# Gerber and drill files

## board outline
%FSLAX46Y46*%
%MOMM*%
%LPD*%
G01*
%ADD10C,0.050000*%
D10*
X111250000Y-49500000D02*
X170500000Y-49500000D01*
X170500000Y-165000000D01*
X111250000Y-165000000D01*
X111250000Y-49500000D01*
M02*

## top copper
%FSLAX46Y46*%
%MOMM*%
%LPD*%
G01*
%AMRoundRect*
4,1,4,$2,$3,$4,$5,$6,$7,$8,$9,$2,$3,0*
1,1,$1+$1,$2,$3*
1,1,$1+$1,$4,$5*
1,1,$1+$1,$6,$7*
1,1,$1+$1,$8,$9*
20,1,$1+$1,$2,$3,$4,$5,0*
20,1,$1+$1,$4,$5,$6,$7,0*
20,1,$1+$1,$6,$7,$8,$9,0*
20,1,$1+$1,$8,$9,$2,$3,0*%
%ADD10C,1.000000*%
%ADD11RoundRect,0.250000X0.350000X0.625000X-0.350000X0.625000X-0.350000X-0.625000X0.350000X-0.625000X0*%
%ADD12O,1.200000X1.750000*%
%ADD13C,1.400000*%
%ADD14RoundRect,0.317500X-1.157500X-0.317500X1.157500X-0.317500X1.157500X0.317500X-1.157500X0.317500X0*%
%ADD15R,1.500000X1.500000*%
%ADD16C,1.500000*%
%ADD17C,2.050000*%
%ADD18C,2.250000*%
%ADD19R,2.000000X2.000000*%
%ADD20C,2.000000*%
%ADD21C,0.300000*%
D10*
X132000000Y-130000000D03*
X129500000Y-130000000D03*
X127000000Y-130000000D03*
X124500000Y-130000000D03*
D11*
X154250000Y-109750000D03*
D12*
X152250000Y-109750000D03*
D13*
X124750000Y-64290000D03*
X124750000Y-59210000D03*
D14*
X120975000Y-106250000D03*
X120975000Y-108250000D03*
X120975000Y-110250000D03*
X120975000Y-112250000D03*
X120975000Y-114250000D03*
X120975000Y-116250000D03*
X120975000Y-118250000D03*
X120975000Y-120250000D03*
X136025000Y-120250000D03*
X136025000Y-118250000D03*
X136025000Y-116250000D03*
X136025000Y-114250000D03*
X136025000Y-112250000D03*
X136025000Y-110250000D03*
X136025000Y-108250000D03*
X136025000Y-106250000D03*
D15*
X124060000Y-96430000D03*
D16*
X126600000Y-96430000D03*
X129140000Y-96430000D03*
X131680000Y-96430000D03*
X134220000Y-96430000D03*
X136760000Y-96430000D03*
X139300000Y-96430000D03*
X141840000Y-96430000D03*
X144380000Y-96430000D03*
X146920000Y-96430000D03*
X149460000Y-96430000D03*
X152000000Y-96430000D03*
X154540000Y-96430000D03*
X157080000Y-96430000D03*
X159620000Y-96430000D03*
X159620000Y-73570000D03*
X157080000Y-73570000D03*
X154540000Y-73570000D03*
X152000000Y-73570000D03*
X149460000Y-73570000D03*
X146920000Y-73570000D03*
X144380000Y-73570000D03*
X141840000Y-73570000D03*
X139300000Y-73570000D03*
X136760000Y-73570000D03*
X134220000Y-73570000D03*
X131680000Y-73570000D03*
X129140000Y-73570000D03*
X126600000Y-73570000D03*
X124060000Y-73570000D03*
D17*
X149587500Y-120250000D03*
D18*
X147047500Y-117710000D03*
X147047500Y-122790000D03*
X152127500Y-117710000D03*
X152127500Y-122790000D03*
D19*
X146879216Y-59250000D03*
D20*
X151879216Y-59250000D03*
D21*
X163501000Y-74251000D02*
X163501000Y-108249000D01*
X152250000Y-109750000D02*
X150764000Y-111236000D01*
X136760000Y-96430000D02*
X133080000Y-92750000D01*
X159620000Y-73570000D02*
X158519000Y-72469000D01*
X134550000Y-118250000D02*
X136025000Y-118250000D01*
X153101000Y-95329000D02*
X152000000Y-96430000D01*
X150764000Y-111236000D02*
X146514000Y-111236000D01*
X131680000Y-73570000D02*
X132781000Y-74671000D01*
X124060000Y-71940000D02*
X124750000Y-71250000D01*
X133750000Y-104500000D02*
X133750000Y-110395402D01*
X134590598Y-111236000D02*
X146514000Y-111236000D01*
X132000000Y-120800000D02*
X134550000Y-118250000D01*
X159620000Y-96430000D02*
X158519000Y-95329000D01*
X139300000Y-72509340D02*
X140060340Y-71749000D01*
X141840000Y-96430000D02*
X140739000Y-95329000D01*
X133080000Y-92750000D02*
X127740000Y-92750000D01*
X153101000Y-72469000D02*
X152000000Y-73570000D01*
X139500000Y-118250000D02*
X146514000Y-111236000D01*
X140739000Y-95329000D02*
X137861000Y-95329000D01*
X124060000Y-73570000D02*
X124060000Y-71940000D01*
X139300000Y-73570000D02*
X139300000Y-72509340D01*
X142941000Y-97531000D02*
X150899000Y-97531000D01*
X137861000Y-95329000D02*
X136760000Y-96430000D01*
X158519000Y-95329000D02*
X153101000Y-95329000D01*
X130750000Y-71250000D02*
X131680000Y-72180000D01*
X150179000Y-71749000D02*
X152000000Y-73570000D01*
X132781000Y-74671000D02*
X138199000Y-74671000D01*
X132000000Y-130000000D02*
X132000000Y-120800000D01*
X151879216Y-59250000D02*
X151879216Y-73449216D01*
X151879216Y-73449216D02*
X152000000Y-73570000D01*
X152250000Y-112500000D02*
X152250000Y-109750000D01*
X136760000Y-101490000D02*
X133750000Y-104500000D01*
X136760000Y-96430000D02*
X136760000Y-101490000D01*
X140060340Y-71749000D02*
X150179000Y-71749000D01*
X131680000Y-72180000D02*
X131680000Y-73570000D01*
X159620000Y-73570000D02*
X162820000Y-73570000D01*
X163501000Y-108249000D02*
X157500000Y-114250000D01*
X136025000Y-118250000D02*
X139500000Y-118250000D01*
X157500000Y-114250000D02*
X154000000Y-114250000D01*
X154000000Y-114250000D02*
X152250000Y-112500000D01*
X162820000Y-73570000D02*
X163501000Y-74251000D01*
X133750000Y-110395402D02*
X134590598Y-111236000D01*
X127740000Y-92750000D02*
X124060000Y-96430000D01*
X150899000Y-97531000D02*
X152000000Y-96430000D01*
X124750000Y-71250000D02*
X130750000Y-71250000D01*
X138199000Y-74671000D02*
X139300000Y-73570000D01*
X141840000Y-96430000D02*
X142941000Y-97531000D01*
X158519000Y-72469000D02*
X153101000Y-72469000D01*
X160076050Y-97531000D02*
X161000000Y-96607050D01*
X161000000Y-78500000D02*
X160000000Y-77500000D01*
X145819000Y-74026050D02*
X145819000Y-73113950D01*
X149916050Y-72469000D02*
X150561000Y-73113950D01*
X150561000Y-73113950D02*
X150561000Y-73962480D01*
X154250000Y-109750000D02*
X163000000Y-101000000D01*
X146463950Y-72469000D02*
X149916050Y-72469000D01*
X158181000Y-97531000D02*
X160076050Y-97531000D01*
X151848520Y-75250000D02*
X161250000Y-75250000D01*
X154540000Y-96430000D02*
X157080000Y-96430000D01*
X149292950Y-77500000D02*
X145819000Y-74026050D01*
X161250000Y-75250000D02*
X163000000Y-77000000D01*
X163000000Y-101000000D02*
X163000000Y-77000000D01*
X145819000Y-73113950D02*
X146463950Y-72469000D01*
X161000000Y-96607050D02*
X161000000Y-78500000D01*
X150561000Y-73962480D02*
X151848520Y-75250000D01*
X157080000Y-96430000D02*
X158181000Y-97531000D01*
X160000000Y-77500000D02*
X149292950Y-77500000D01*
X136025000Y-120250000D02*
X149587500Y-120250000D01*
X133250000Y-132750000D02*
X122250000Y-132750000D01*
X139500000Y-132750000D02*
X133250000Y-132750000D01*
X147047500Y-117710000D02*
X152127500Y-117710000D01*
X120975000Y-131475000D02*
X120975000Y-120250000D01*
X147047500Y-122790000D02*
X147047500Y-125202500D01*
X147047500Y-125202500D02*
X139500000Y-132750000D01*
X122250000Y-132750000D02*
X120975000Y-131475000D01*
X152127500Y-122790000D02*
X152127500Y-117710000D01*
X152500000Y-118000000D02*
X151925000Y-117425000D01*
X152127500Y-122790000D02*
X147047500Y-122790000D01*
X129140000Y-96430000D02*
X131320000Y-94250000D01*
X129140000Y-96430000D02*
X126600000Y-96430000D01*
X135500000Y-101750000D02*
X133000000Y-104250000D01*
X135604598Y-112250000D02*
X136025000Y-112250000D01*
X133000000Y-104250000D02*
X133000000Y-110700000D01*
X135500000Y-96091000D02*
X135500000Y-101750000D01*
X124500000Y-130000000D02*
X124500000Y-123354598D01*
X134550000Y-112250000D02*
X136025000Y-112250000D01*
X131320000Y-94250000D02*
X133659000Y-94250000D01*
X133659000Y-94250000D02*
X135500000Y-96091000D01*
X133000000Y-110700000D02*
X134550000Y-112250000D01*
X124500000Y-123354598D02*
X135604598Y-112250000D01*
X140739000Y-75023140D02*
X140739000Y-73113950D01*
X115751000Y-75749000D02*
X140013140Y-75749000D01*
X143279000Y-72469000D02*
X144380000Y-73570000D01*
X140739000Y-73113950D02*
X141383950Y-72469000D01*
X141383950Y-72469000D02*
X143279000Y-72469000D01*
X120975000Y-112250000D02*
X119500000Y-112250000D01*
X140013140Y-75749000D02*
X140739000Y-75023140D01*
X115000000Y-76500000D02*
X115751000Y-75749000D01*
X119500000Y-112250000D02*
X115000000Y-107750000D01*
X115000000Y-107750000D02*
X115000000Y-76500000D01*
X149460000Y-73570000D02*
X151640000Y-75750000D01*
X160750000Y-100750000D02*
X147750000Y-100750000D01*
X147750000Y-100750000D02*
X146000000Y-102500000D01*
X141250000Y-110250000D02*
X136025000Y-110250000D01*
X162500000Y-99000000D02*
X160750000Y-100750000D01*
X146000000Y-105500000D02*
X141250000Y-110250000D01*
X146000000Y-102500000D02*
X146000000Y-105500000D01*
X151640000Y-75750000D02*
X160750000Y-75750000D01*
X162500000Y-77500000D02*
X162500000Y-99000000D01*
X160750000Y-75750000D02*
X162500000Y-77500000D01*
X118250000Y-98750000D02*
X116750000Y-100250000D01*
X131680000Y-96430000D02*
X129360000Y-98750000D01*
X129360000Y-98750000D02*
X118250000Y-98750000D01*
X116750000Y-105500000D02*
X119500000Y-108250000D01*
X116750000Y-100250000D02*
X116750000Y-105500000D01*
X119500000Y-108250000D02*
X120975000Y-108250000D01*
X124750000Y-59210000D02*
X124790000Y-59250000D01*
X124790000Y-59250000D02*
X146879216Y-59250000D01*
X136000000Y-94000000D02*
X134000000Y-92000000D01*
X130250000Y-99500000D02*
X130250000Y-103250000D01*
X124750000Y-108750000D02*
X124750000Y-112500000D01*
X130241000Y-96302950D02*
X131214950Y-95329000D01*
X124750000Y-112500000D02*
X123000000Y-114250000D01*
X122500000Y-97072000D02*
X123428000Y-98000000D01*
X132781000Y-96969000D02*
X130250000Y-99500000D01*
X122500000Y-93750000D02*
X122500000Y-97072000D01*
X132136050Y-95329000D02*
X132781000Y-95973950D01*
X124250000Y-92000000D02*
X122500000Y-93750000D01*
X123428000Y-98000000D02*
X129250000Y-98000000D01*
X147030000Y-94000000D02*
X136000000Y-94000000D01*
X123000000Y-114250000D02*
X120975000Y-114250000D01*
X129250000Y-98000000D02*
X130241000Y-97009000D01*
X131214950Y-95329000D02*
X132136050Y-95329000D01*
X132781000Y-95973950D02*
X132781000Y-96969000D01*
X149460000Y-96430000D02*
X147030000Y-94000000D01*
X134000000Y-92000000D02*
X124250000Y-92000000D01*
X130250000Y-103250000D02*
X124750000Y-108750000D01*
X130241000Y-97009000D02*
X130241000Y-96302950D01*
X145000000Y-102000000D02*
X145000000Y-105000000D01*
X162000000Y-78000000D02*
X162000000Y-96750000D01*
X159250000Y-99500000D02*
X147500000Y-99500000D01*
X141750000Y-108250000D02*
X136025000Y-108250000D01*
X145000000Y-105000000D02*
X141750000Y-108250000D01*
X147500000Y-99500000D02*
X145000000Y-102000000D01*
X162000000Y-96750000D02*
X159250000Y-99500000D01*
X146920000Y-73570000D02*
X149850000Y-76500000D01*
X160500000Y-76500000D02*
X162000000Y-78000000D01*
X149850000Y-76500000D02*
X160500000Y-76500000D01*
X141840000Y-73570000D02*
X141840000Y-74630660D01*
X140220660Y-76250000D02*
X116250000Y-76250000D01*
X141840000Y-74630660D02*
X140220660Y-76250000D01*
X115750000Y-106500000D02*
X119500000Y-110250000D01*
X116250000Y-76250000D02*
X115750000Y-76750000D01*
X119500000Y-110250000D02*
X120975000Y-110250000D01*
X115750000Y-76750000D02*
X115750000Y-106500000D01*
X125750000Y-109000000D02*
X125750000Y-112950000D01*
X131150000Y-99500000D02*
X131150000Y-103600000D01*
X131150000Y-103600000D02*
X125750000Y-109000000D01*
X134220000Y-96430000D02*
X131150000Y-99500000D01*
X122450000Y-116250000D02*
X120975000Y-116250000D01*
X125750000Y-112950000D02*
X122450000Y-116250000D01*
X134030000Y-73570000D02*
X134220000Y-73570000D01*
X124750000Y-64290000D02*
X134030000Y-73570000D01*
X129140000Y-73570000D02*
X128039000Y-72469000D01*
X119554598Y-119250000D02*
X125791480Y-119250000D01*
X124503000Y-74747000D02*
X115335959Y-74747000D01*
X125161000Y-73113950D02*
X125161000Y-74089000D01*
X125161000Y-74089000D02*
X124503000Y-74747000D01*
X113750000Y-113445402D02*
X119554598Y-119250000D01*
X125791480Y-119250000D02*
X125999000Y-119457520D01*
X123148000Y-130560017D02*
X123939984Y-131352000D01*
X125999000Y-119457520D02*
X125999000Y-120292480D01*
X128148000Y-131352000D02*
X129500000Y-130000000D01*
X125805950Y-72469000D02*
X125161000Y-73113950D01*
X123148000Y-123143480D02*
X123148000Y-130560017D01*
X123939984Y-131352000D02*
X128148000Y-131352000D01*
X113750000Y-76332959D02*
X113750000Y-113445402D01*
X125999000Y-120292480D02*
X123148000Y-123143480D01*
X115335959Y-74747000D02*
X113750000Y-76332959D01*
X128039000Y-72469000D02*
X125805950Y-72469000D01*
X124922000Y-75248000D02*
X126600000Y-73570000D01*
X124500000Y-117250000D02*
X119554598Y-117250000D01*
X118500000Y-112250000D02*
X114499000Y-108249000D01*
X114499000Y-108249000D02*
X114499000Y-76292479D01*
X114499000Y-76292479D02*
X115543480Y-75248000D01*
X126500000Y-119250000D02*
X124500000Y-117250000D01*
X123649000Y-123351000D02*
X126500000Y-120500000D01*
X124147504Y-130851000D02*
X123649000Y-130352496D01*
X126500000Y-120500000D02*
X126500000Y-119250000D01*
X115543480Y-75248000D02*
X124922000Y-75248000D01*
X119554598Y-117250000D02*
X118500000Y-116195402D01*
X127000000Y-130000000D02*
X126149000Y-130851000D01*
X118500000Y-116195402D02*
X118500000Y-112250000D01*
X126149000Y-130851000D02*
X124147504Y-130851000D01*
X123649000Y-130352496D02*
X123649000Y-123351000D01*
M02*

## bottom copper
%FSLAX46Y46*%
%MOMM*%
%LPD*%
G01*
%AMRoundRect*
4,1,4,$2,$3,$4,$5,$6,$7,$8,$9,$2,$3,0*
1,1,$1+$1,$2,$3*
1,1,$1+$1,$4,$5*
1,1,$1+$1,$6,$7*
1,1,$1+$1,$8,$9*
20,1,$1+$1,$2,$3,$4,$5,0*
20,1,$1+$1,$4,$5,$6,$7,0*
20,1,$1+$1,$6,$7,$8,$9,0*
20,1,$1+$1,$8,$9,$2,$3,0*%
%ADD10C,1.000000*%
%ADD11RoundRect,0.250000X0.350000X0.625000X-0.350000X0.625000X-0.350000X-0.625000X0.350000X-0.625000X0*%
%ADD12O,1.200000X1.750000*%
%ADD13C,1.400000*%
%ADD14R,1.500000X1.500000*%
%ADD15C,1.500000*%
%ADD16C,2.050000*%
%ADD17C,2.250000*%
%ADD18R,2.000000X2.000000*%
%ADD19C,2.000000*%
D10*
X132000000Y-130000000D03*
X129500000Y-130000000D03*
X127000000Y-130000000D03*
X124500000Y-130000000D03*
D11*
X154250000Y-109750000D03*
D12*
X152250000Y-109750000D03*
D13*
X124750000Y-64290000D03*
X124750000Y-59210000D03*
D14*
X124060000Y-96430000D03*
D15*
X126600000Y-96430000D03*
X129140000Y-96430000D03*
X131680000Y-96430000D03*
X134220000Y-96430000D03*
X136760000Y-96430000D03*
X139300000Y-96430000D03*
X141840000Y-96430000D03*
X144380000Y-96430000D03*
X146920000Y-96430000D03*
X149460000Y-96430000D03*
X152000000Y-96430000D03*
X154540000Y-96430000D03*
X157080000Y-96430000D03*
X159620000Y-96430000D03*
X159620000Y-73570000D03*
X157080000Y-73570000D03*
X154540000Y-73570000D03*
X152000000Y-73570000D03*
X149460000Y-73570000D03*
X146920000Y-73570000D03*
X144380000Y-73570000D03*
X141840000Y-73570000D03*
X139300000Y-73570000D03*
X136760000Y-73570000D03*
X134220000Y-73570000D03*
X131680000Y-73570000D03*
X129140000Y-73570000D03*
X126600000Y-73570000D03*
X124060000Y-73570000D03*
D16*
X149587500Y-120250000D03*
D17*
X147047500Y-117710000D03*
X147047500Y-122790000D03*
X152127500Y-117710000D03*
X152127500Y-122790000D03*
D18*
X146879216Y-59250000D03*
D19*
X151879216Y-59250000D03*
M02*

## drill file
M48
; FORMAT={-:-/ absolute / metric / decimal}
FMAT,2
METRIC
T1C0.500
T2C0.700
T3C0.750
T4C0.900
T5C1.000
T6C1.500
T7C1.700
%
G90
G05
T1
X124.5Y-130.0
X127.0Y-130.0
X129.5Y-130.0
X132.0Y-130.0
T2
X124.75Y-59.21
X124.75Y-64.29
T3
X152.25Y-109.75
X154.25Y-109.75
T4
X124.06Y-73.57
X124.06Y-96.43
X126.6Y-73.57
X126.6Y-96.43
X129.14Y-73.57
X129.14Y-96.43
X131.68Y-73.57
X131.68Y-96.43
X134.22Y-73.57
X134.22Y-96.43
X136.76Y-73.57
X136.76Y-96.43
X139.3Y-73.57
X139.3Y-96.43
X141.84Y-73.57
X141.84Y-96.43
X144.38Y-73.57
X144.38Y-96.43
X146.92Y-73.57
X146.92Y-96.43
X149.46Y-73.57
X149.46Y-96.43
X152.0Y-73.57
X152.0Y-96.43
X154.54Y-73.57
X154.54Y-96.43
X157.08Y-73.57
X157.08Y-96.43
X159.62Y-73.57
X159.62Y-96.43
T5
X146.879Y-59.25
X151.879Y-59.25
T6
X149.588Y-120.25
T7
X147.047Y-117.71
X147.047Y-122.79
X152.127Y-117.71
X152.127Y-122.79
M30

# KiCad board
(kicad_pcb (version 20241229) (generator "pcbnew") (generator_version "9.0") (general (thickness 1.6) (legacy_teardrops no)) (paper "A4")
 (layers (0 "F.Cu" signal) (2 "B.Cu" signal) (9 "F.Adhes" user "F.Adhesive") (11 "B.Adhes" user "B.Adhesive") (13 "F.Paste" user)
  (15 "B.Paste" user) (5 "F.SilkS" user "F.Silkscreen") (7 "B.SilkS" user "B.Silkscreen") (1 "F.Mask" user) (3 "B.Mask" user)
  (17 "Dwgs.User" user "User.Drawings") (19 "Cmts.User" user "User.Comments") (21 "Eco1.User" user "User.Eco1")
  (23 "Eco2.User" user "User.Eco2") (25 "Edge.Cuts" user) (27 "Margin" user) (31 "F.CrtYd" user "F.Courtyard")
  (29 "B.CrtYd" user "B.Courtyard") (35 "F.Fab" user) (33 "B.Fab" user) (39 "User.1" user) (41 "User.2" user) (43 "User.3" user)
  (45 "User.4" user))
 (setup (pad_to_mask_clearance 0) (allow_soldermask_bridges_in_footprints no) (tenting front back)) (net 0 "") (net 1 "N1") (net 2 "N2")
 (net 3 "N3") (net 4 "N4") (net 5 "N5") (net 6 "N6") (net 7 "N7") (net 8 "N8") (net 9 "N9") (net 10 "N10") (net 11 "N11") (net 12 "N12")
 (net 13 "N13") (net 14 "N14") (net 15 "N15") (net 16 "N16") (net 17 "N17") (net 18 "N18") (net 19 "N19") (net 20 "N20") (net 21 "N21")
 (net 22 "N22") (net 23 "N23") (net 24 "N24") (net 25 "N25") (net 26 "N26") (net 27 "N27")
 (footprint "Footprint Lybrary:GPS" (layer "F.Cu") (at 136 147.5 -90)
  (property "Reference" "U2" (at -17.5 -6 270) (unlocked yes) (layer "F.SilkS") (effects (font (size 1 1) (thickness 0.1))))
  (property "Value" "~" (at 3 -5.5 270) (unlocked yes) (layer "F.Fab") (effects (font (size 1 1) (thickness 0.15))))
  (pad "1" thru_hole circle (at -17.5 4 270) (size 1 1) (drill 0.5) (layers "*.Cu" "*.Mask") (remove_unused_layers no) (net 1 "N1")
   (solder_mask_margin 0.102))
  (pad "2" thru_hole circle (at -17.5 6.5 270) (size 1 1) (drill 0.5) (layers "*.Cu" "*.Mask") (remove_unused_layers no) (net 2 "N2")
   (solder_mask_margin 0.102))
  (pad "3" thru_hole circle (at -17.5 9 270) (size 1 1) (drill 0.5) (layers "*.Cu" "*.Mask") (remove_unused_layers no) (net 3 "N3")
   (solder_mask_margin 0.102))
  (pad "4" thru_hole circle (at -17.5 11.5 270) (size 1 1) (drill 0.5) (layers "*.Cu" "*.Mask") (remove_unused_layers no) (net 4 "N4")
   (solder_mask_margin 0.102))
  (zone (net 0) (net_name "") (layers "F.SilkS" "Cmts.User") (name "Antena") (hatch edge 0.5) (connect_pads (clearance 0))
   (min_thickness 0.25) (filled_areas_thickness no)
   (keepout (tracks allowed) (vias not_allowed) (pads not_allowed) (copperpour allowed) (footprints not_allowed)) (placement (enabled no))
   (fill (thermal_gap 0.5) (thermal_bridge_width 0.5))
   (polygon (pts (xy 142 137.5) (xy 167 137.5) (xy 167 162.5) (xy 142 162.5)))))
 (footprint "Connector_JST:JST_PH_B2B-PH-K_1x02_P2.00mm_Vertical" (layer "F.Cu") (at 154.25 109.75 180)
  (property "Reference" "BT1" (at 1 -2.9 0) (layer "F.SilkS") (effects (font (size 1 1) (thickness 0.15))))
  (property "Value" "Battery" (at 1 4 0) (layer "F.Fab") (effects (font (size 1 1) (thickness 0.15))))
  (pad "1" thru_hole roundrect (at 0 0 180) (size 1.2 1.75) (drill 0.75) (layers "*.Cu" "*.Mask") (remove_unused_layers no)
   (roundrect_rratio 0.208333) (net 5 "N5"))
  (pad "2" thru_hole oval (at 2 0 180) (size 1.2 1.75) (drill 0.75) (layers "*.Cu" "*.Mask") (remove_unused_layers no) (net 1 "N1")))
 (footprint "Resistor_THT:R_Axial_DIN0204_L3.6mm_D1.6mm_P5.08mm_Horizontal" (layer "F.Cu") (at 124.75 64.29 90)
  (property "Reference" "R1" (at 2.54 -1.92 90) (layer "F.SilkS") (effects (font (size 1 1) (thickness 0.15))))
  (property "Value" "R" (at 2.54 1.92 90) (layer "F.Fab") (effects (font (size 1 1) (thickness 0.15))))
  (pad "1" thru_hole circle (at 0 0 90) (size 1.4 1.4) (drill 0.7) (layers "*.Cu" "*.Mask") (remove_unused_layers no) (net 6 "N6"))
  (pad "2" thru_hole circle (at 5.08 0 90) (size 1.4 1.4) (drill 0.7) (layers "*.Cu" "*.Mask") (remove_unused_layers no) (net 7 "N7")))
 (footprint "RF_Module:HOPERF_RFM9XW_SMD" (layer "F.Cu") (at 128.5 113.25)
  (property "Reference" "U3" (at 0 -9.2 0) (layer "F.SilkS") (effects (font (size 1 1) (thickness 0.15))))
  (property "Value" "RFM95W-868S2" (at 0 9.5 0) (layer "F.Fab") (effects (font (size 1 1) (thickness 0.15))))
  (pad "1" smd roundrect (at -7.525 -7) (size 2.95 1.27) (layers "F.Cu" "F.Mask" "F.Paste") (roundrect_rratio 0.25) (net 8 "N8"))
  (pad "2" smd roundrect (at -7.525 -5) (size 2.95 1.27) (layers "F.Cu" "F.Mask" "F.Paste") (roundrect_rratio 0.25) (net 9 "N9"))
  (pad "3" smd roundrect (at -7.525 -3) (size 2.95 1.27) (layers "F.Cu" "F.Mask" "F.Paste") (roundrect_rratio 0.25) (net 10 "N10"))
  (pad "4" smd roundrect (at -7.525 -1) (size 2.95 1.27) (layers "F.Cu" "F.Mask" "F.Paste") (roundrect_rratio 0.25) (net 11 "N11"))
  (pad "5" smd roundrect (at -7.525 1) (size 2.95 1.27) (layers "F.Cu" "F.Mask" "F.Paste") (roundrect_rratio 0.25) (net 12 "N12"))
  (pad "6" smd roundrect (at -7.525 3) (size 2.95 1.27) (layers "F.Cu" "F.Mask" "F.Paste") (roundrect_rratio 0.25) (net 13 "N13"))
  (pad "7" smd roundrect (at -7.525 5) (size 2.95 1.27) (layers "F.Cu" "F.Mask" "F.Paste") (roundrect_rratio 0.25) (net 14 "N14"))
  (pad "8" smd roundrect (at -7.525 7) (size 2.95 1.27) (layers "F.Cu" "F.Mask" "F.Paste") (roundrect_rratio 0.25) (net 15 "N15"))
  (pad "9" smd roundrect (at 7.525 7) (size 2.95 1.27) (layers "F.Cu" "F.Mask" "F.Paste") (roundrect_rratio 0.25) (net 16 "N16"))
  (pad "10" smd roundrect (at 7.525 5) (size 2.95 1.27) (layers "F.Cu" "F.Mask" "F.Paste") (roundrect_rratio 0.25) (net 1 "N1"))
  (pad "11" smd roundrect (at 7.525 3) (size 2.95 1.27) (layers "F.Cu" "F.Mask" "F.Paste") (roundrect_rratio 0.25) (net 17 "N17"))
  (pad "12" smd roundrect (at 7.525 1) (size 2.95 1.27) (layers "F.Cu" "F.Mask" "F.Paste") (roundrect_rratio 0.25) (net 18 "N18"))
  (pad "13" smd roundrect (at 7.525 -1) (size 2.95 1.27) (layers "F.Cu" "F.Mask" "F.Paste") (roundrect_rratio 0.25) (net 4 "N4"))
  (pad "14" smd roundrect (at 7.525 -3) (size 2.95 1.27) (layers "F.Cu" "F.Mask" "F.Paste") (roundrect_rratio 0.25) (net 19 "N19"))
  (pad "15" smd roundrect (at 7.525 -5) (size 2.95 1.27) (layers "F.Cu" "F.Mask" "F.Paste") (roundrect_rratio 0.25) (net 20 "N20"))
  (pad "16" smd roundrect (at 7.525 -7) (size 2.95 1.27) (layers "F.Cu" "F.Mask" "F.Paste") (roundrect_rratio 0.25) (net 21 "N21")))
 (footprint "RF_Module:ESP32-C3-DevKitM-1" (layer "F.Cu") (at 124.06 96.43 90)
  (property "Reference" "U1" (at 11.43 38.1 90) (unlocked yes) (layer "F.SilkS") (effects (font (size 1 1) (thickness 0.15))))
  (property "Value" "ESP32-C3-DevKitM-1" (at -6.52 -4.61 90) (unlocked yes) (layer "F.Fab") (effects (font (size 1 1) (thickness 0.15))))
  (pad "1" thru_hole rect (at 0 0 90) (size 1.5 1.5) (drill 0.9) (layers "*.Cu" "*.Mask") (remove_unused_layers yes) (keep_end_layers yes)
   (zone_layer_connections) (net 1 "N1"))
  (pad "2" thru_hole circle (at 0 2.54 90) (size 1.5 1.5) (drill 0.9) (layers "*.Cu" "*.Mask") (remove_unused_layers yes)
   (keep_end_layers yes) (zone_layer_connections) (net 4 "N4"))
  (pad "3" thru_hole circle (at 0 5.08 90) (size 1.5 1.5) (drill 0.9) (layers "*.Cu" "*.Mask") (remove_unused_layers yes)
   (keep_end_layers yes) (zone_layer_connections) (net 4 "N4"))
  (pad "4" thru_hole circle (at 0 7.62 90) (size 1.5 1.5) (drill 0.9) (layers "*.Cu" "*.Mask") (remove_unused_layers yes)
   (keep_end_layers yes) (zone_layer_connections) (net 9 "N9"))
  (pad "5" thru_hole circle (at 0 10.16 90) (size 1.5 1.5) (drill 0.9) (layers "*.Cu" "*.Mask") (remove_unused_layers yes)
   (keep_end_layers yes) (zone_layer_connections) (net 13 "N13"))
  (pad "6" thru_hole circle (at 0 12.7 90) (size 1.5 1.5) (drill 0.9) (layers "*.Cu" "*.Mask") (remove_unused_layers yes)
   (keep_end_layers yes) (zone_layer_connections) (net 1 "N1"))
  (pad "7" thru_hole circle (at 0 15.24 90) (size 1.5 1.5) (drill 0.9) (layers "*.Cu" "*.Mask") (remove_unused_layers yes)
   (keep_end_layers yes) (zone_layer_connections) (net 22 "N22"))
  (pad "8" thru_hole circle (at 0 17.78 90) (size 1.5 1.5) (drill 0.9) (layers "*.Cu" "*.Mask") (remove_unused_layers yes)
   (keep_end_layers yes) (zone_layer_connections) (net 1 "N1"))
  (pad "9" thru_hole circle (at 0 20.32 90) (size 1.5 1.5) (drill 0.9) (layers "*.Cu" "*.Mask") (remove_unused_layers yes)
   (keep_end_layers yes) (zone_layer_connections) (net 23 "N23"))
  (pad "10" thru_hole circle (at 0 22.86 90) (size 1.5 1.5) (drill 0.9) (layers "*.Cu" "*.Mask") (remove_unused_layers yes)
   (keep_end_layers yes) (zone_layer_connections) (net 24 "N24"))
  (pad "11" thru_hole circle (at 0 25.4 90) (size 1.5 1.5) (drill 0.9) (layers "*.Cu" "*.Mask") (remove_unused_layers yes)
   (keep_end_layers yes) (zone_layer_connections) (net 12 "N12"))
  (pad "12" thru_hole circle (at 0 27.94 90) (size 1.5 1.5) (drill 0.9) (layers "*.Cu" "*.Mask") (remove_unused_layers yes)
   (keep_end_layers yes) (zone_layer_connections) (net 1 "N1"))
  (pad "13" thru_hole circle (at 0 30.48 90) (size 1.5 1.5) (drill 0.9) (layers "*.Cu" "*.Mask") (remove_unused_layers yes)
   (keep_end_layers yes) (zone_layer_connections) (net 5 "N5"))
  (pad "14" thru_hole circle (at 0 33.02 90) (size 1.5 1.5) (drill 0.9) (layers "*.Cu" "*.Mask") (remove_unused_layers yes)
   (keep_end_layers yes) (zone_layer_connections) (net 5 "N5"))
  (pad "15" thru_hole circle (at 0 35.56 90) (size 1.5 1.5) (drill 0.9) (layers "*.Cu" "*.Mask") (remove_unused_layers yes)
   (keep_end_layers yes) (zone_layer_connections) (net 1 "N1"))
  (pad "16" thru_hole circle (at 22.86 35.56 90) (size 1.5 1.5) (drill 0.9) (layers "*.Cu" "*.Mask") (remove_unused_layers yes)
   (keep_end_layers yes) (zone_layer_connections) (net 1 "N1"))
  (pad "17" thru_hole circle (at 22.86 33.02 90) (size 1.5 1.5) (drill 0.9) (layers "*.Cu" "*.Mask") (remove_unused_layers yes)
   (keep_end_layers yes) (zone_layer_connections) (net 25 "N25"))
  (pad "18" thru_hole circle (at 22.86 30.48 90) (size 1.5 1.5) (drill 0.9) (layers "*.Cu" "*.Mask") (remove_unused_layers yes)
   (keep_end_layers yes) (zone_layer_connections) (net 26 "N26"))
  (pad "19" thru_hole circle (at 22.86 27.94 90) (size 1.5 1.5) (drill 0.9) (layers "*.Cu" "*.Mask") (remove_unused_layers yes)
   (keep_end_layers yes) (zone_layer_connections) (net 1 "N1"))
  (pad "20" thru_hole circle (at 22.86 25.4 90) (size 1.5 1.5) (drill 0.9) (layers "*.Cu" "*.Mask") (remove_unused_layers yes)
   (keep_end_layers yes) (zone_layer_connections) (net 19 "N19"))
  (pad "21" thru_hole circle (at 22.86 22.86 90) (size 1.5 1.5) (drill 0.9) (layers "*.Cu" "*.Mask") (remove_unused_layers yes)
   (keep_end_layers yes) (zone_layer_connections) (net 20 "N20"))
  (pad "22" thru_hole circle (at 22.86 20.32 90) (size 1.5 1.5) (drill 0.9) (layers "*.Cu" "*.Mask") (remove_unused_layers yes)
   (keep_end_layers yes) (zone_layer_connections) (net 11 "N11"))
  (pad "23" thru_hole circle (at 22.86 17.78 90) (size 1.5 1.5) (drill 0.9) (layers "*.Cu" "*.Mask") (remove_unused_layers yes)
   (keep_end_layers yes) (zone_layer_connections) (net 10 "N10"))
  (pad "24" thru_hole circle (at 22.86 15.24 90) (size 1.5 1.5) (drill 0.9) (layers "*.Cu" "*.Mask") (remove_unused_layers yes)
   (keep_end_layers yes) (zone_layer_connections) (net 1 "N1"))
  (pad "25" thru_hole circle (at 22.86 12.7 90) (size 1.5 1.5) (drill 0.9) (layers "*.Cu" "*.Mask") (remove_unused_layers yes)
   (keep_end_layers yes) (zone_layer_connections) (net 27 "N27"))
  (pad "26" thru_hole circle (at 22.86 10.16 90) (size 1.5 1.5) (drill 0.9) (layers "*.Cu" "*.Mask") (remove_unused_layers yes)
   (keep_end_layers yes) (zone_layer_connections) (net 6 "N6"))
  (pad "27" thru_hole circle (at 22.86 7.62 90) (size 1.5 1.5) (drill 0.9) (layers "*.Cu" "*.Mask") (remove_unused_layers yes)
   (keep_end_layers yes) (zone_layer_connections) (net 1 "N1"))
  (pad "28" thru_hole circle (at 22.86 5.08 90) (size 1.5 1.5) (drill 0.9) (layers "*.Cu" "*.Mask") (remove_unused_layers yes)
   (keep_end_layers yes) (zone_layer_connections) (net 2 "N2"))
  (pad "29" thru_hole circle (at 22.86 2.54 90) (size 1.5 1.5) (drill 0.9) (layers "*.Cu" "*.Mask") (remove_unused_layers yes)
   (keep_end_layers yes) (zone_layer_connections) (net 3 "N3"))
  (pad "30" thru_hole circle (at 22.86 0 90) (size 1.5 1.5) (drill 0.9) (layers "*.Cu" "*.Mask") (remove_unused_layers yes)
   (keep_end_layers yes) (zone_layer_connections) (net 1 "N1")))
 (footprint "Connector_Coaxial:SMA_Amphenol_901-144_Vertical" (layer "F.Cu") (at 149.5875 120.25)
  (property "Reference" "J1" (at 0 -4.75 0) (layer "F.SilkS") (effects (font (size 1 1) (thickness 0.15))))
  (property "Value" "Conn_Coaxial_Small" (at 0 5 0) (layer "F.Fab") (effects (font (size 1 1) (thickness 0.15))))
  (pad "1" thru_hole circle (at 0 0) (size 2.05 2.05) (drill 1.5) (layers "*.Cu" "*.Mask") (remove_unused_layers no) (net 16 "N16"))
  (pad "2" thru_hole circle (at -2.54 -2.54) (size 2.25 2.25) (drill 1.7) (layers "*.Cu" "*.Mask") (remove_unused_layers no) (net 15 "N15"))
  (pad "2" thru_hole circle (at -2.54 2.54) (size 2.25 2.25) (drill 1.7) (layers "*.Cu" "*.Mask") (remove_unused_layers no) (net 15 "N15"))
  (pad "2" thru_hole circle (at 2.54 -2.54) (size 2.25 2.25) (drill 1.7) (layers "*.Cu" "*.Mask") (remove_unused_layers no) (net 15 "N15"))
  (pad "2" thru_hole circle (at 2.54 2.54) (size 2.25 2.25) (drill 1.7) (layers "*.Cu" "*.Mask") (remove_unused_layers no) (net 15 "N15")))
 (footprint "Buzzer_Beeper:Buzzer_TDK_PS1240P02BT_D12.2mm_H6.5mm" (layer "F.Cu") (at 146.879216 59.25)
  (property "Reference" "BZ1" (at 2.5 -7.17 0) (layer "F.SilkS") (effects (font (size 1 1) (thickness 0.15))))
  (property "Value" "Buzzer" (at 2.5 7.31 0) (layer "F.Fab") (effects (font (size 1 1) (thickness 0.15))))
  (pad "1" thru_hole rect (at 0 0) (size 2 2) (drill 1) (layers "*.Cu" "*.Mask") (remove_unused_layers no) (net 7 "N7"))
  (pad "2" thru_hole circle (at 5 0) (size 2 2) (drill 1) (layers "*.Cu" "*.Mask") (remove_unused_layers no) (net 1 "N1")))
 (gr_rect (start 111.25 49.5) (end 170.5 165) (stroke (width 0.05) (type default)) (fill no) (layer "Edge.Cuts"))
 (segment (start 163.501 74.251) (end 163.501 108.249) (width 0.3) (layer "F.Cu") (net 1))
 (segment (start 152.25 109.75) (end 150.764 111.236) (width 0.3) (layer "F.Cu") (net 1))
 (segment (start 136.76 96.43) (end 133.08 92.75) (width 0.3) (layer "F.Cu") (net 1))
 (segment (start 159.62 73.57) (end 158.519 72.469) (width 0.3) (layer "F.Cu") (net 1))
 (segment (start 134.55 118.25) (end 136.025 118.25) (width 0.3) (layer "F.Cu") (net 1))
 (segment (start 153.101 95.329) (end 152 96.43) (width 0.3) (layer "F.Cu") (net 1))
 (segment (start 150.764 111.236) (end 146.514 111.236) (width 0.3) (layer "F.Cu") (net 1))
 (segment (start 131.68 73.57) (end 132.781 74.671) (width 0.3) (layer "F.Cu") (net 1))
 (segment (start 124.06 71.94) (end 124.75 71.25) (width 0.3) (layer "F.Cu") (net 1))
 (segment (start 133.75 104.5) (end 133.75 110.395402) (width 0.3) (layer "F.Cu") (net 1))
 (segment (start 134.590598 111.236) (end 146.514 111.236) (width 0.3) (layer "F.Cu") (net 1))
 (segment (start 132 120.8) (end 134.55 118.25) (width 0.3) (layer "F.Cu") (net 1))
 (segment (start 159.62 96.43) (end 158.519 95.329) (width 0.3) (layer "F.Cu") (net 1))
 (segment (start 139.3 72.50934) (end 140.06034 71.749) (width 0.3) (layer "F.Cu") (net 1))
 (segment (start 141.84 96.43) (end 140.739 95.329) (width 0.3) (layer "F.Cu") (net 1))
 (segment (start 133.08 92.75) (end 127.74 92.75) (width 0.3) (layer "F.Cu") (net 1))
 (segment (start 153.101 72.469) (end 152 73.57) (width 0.3) (layer "F.Cu") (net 1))
 (segment (start 139.5 118.25) (end 146.514 111.236) (width 0.3) (layer "F.Cu") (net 1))
 (segment (start 140.739 95.329) (end 137.861 95.329) (width 0.3) (layer "F.Cu") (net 1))
 (segment (start 124.06 73.57) (end 124.06 71.94) (width 0.3) (layer "F.Cu") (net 1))
 (segment (start 139.3 73.57) (end 139.3 72.50934) (width 0.3) (layer "F.Cu") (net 1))
 (segment (start 142.941 97.531) (end 150.899 97.531) (width 0.3) (layer "F.Cu") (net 1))
 (segment (start 137.861 95.329) (end 136.76 96.43) (width 0.3) (layer "F.Cu") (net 1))
 (segment (start 158.519 95.329) (end 153.101 95.329) (width 0.3) (layer "F.Cu") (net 1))
 (segment (start 130.75 71.25) (end 131.68 72.18) (width 0.3) (layer "F.Cu") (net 1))
 (segment (start 150.179 71.749) (end 152 73.57) (width 0.3) (layer "F.Cu") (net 1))
 (segment (start 132.781 74.671) (end 138.199 74.671) (width 0.3) (layer "F.Cu") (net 1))
 (segment (start 132 130) (end 132 120.8) (width 0.3) (layer "F.Cu") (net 1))
 (segment (start 151.879216 59.25) (end 151.879216 73.449216) (width 0.3) (layer "F.Cu") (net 1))
 (segment (start 151.879216 73.449216) (end 152 73.57) (width 0.3) (layer "F.Cu") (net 1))
 (segment (start 152.25 112.5) (end 152.25 109.75) (width 0.3) (layer "F.Cu") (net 1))
 (segment (start 136.76 101.49) (end 133.75 104.5) (width 0.3) (layer "F.Cu") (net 1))
 (segment (start 136.76 96.43) (end 136.76 101.49) (width 0.3) (layer "F.Cu") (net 1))
 (segment (start 140.06034 71.749) (end 150.179 71.749) (width 0.3) (layer "F.Cu") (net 1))
 (segment (start 131.68 72.18) (end 131.68 73.57) (width 0.3) (layer "F.Cu") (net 1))
 (segment (start 159.62 73.57) (end 162.82 73.57) (width 0.3) (layer "F.Cu") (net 1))
 (segment (start 163.501 108.249) (end 157.5 114.25) (width 0.3) (layer "F.Cu") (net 1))
 (segment (start 136.025 118.25) (end 139.5 118.25) (width 0.3) (layer "F.Cu") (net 1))
 (segment (start 157.5 114.25) (end 154 114.25) (width 0.3) (layer "F.Cu") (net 1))
 (segment (start 154 114.25) (end 152.25 112.5) (width 0.3) (layer "F.Cu") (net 1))
 (segment (start 162.82 73.57) (end 163.501 74.251) (width 0.3) (layer "F.Cu") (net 1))
 (segment (start 133.75 110.395402) (end 134.590598 111.236) (width 0.3) (layer "F.Cu") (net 1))
 (segment (start 127.74 92.75) (end 124.06 96.43) (width 0.3) (layer "F.Cu") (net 1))
 (segment (start 150.899 97.531) (end 152 96.43) (width 0.3) (layer "F.Cu") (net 1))
 (segment (start 124.75 71.25) (end 130.75 71.25) (width 0.3) (layer "F.Cu") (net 1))
 (segment (start 138.199 74.671) (end 139.3 73.57) (width 0.3) (layer "F.Cu") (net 1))
 (segment (start 141.84 96.43) (end 142.941 97.531) (width 0.3) (layer "F.Cu") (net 1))
 (segment (start 158.519 72.469) (end 153.101 72.469) (width 0.3) (layer "F.Cu") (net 1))
 (segment (start 160.07605 97.531) (end 161 96.60705) (width 0.3) (layer "F.Cu") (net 5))
 (segment (start 161 78.5) (end 160 77.5) (width 0.3) (layer "F.Cu") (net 5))
 (segment (start 145.819 74.02605) (end 145.819 73.11395) (width 0.3) (layer "F.Cu") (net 5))
 (segment (start 149.91605 72.469) (end 150.561 73.11395) (width 0.3) (layer "F.Cu") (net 5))
 (segment (start 150.561 73.11395) (end 150.561 73.96248) (width 0.3) (layer "F.Cu") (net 5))
 (segment (start 154.25 109.75) (end 163 101) (width 0.3) (layer "F.Cu") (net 5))
 (segment (start 146.46395 72.469) (end 149.91605 72.469) (width 0.3) (layer "F.Cu") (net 5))
 (segment (start 158.181 97.531) (end 160.07605 97.531) (width 0.3) (layer "F.Cu") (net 5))
 (segment (start 151.84852 75.25) (end 161.25 75.25) (width 0.3) (layer "F.Cu") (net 5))
 (segment (start 154.54 96.43) (end 157.08 96.43) (width 0.3) (layer "F.Cu") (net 5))
 (segment (start 149.29295 77.5) (end 145.819 74.02605) (width 0.3) (layer "F.Cu") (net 5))
 (segment (start 161.25 75.25) (end 163 77) (width 0.3) (layer "F.Cu") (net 5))
 (segment (start 163 101) (end 163 77) (width 0.3) (layer "F.Cu") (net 5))
 (segment (start 145.819 73.11395) (end 146.46395 72.469) (width 0.3) (layer "F.Cu") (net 5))
 (segment (start 161 96.60705) (end 161 78.5) (width 0.3) (layer "F.Cu") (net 5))
 (segment (start 150.561 73.96248) (end 151.84852 75.25) (width 0.3) (layer "F.Cu") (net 5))
 (segment (start 157.08 96.43) (end 158.181 97.531) (width 0.3) (layer "F.Cu") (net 5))
 (segment (start 160 77.5) (end 149.29295 77.5) (width 0.3) (layer "F.Cu") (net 5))
 (segment (start 136.025 120.25) (end 149.5875 120.25) (width 0.3) (layer "F.Cu") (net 16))
 (segment (start 133.25 132.75) (end 122.25 132.75) (width 0.3) (layer "F.Cu") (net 15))
 (segment (start 139.5 132.75) (end 133.25 132.75) (width 0.3) (layer "F.Cu") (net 15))
 (segment (start 147.0475 117.71) (end 152.1275 117.71) (width 0.3) (layer "F.Cu") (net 15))
 (segment (start 120.975 131.475) (end 120.975 120.25) (width 0.3) (layer "F.Cu") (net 15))
 (segment (start 147.0475 122.79) (end 147.0475 125.2025) (width 0.3) (layer "F.Cu") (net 15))
 (segment (start 147.0475 125.2025) (end 139.5 132.75) (width 0.3) (layer "F.Cu") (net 15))
 (segment (start 122.25 132.75) (end 120.975 131.475) (width 0.3) (layer "F.Cu") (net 15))
 (segment (start 152.1275 122.79) (end 152.1275 117.71) (width 0.3) (layer "F.Cu") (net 15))
 (segment (start 152.5 118) (end 151.925 117.425) (width 0.3) (layer "F.Cu") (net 15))
 (segment (start 152.1275 122.79) (end 147.0475 122.79) (width 0.3) (layer "F.Cu") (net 15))
 (segment (start 129.14 96.43) (end 131.32 94.25) (width 0.3) (layer "F.Cu") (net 4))
 (segment (start 129.14 96.43) (end 126.6 96.43) (width 0.3) (layer "F.Cu") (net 4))
 (segment (start 135.5 101.75) (end 133 104.25) (width 0.3) (layer "F.Cu") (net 4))
 (segment (start 135.604598 112.25) (end 136.025 112.25) (width 0.3) (layer "F.Cu") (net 4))
 (segment (start 133 104.25) (end 133 110.7) (width 0.3) (layer "F.Cu") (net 4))
 (segment (start 135.5 96.091) (end 135.5 101.75) (width 0.3) (layer "F.Cu") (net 4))
 (segment (start 124.5 130) (end 124.5 123.354598) (width 0.3) (layer "F.Cu") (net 4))
 (segment (start 134.55 112.25) (end 136.025 112.25) (width 0.3) (layer "F.Cu") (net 4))
 (segment (start 131.32 94.25) (end 133.659 94.25) (width 0.3) (layer "F.Cu") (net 4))
 (segment (start 133.659 94.25) (end 135.5 96.091) (width 0.3) (layer "F.Cu") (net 4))
 (segment (start 133 110.7) (end 134.55 112.25) (width 0.3) (layer "F.Cu") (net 4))
 (segment (start 124.5 123.354598) (end 135.604598 112.25) (width 0.3) (layer "F.Cu") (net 4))
 (segment (start 140.739 75.02314) (end 140.739 73.11395) (width 0.3) (layer "F.Cu") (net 11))
 (segment (start 115.751 75.749) (end 140.01314 75.749) (width 0.3) (layer "F.Cu") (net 11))
 (segment (start 143.279 72.469) (end 144.38 73.57) (width 0.3) (layer "F.Cu") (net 11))
 (segment (start 140.739 73.11395) (end 141.38395 72.469) (width 0.3) (layer "F.Cu") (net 11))
 (segment (start 141.38395 72.469) (end 143.279 72.469) (width 0.3) (layer "F.Cu") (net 11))
 (segment (start 120.975 112.25) (end 119.5 112.25) (width 0.3) (layer "F.Cu") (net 11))
 (segment (start 140.01314 75.749) (end 140.739 75.02314) (width 0.3) (layer "F.Cu") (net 11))
 (segment (start 115 76.5) (end 115.751 75.749) (width 0.3) (layer "F.Cu") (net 11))
 (segment (start 119.5 112.25) (end 115 107.75) (width 0.3) (layer "F.Cu") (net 11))
 (segment (start 115 107.75) (end 115 76.5) (width 0.3) (layer "F.Cu") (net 11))
 (segment (start 149.46 73.57) (end 151.64 75.75) (width 0.3) (layer "F.Cu") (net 19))
 (segment (start 160.75 100.75) (end 147.75 100.75) (width 0.3) (layer "F.Cu") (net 19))
 (segment (start 147.75 100.75) (end 146 102.5) (width 0.3) (layer "F.Cu") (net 19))
 (segment (start 141.25 110.25) (end 136.025 110.25) (width 0.3) (layer "F.Cu") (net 19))
 (segment (start 162.5 99) (end 160.75 100.75) (width 0.3) (layer "F.Cu") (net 19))
 (segment (start 146 105.5) (end 141.25 110.25) (width 0.3) (layer "F.Cu") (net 19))
 (segment (start 146 102.5) (end 146 105.5) (width 0.3) (layer "F.Cu") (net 19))
 (segment (start 151.64 75.75) (end 160.75 75.75) (width 0.3) (layer "F.Cu") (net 19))
 (segment (start 162.5 77.5) (end 162.5 99) (width 0.3) (layer "F.Cu") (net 19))
 (segment (start 160.75 75.75) (end 162.5 77.5) (width 0.3) (layer "F.Cu") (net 19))
 (segment (start 118.25 98.75) (end 116.75 100.25) (width 0.3) (layer "F.Cu") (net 9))
 (segment (start 131.68 96.43) (end 129.36 98.75) (width 0.3) (layer "F.Cu") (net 9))
 (segment (start 129.36 98.75) (end 118.25 98.75) (width 0.3) (layer "F.Cu") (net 9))
 (segment (start 116.75 105.5) (end 119.5 108.25) (width 0.3) (layer "F.Cu") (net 9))
 (segment (start 116.75 100.25) (end 116.75 105.5) (width 0.3) (layer "F.Cu") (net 9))
 (segment (start 119.5 108.25) (end 120.975 108.25) (width 0.3) (layer "F.Cu") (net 9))
 (segment (start 124.75 59.21) (end 124.79 59.25) (width 0.3) (layer "F.Cu") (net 7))
 (segment (start 124.79 59.25) (end 146.879216 59.25) (width 0.3) (layer "F.Cu") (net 7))
 (segment (start 136 94) (end 134 92) (width 0.3) (layer "F.Cu") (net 12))
 (segment (start 130.25 99.5) (end 130.25 103.25) (width 0.3) (layer "F.Cu") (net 12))
 (segment (start 124.75 108.75) (end 124.75 112.5) (width 0.3) (layer "F.Cu") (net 12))
 (segment (start 130.241 96.30295) (end 131.21495 95.329) (width 0.3) (layer "F.Cu") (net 12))
 (segment (start 124.75 112.5) (end 123 114.25) (width 0.3) (layer "F.Cu") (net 12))
 (segment (start 122.5 97.072) (end 123.428 98) (width 0.3) (layer "F.Cu") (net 12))
 (segment (start 132.781 96.969) (end 130.25 99.5) (width 0.3) (layer "F.Cu") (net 12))
 (segment (start 122.5 93.75) (end 122.5 97.072) (width 0.3) (layer "F.Cu") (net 12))
 (segment (start 132.13605 95.329) (end 132.781 95.97395) (width 0.3) (layer "F.Cu") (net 12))
 (segment (start 124.25 92) (end 122.5 93.75) (width 0.3) (layer "F.Cu") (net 12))
 (segment (start 123.428 98) (end 129.25 98) (width 0.3) (layer "F.Cu") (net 12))
 (segment (start 147.03 94) (end 136 94) (width 0.3) (layer "F.Cu") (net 12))
 (segment (start 123 114.25) (end 120.975 114.25) (width 0.3) (layer "F.Cu") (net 12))
 (segment (start 129.25 98) (end 130.241 97.009) (width 0.3) (layer "F.Cu") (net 12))
 (segment (start 131.21495 95.329) (end 132.13605 95.329) (width 0.3) (layer "F.Cu") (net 12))
 (segment (start 132.781 95.97395) (end 132.781 96.969) (width 0.3) (layer "F.Cu") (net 12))
 (segment (start 149.46 96.43) (end 147.03 94) (width 0.3) (layer "F.Cu") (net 12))
 (segment (start 134 92) (end 124.25 92) (width 0.3) (layer "F.Cu") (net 12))
 (segment (start 130.25 103.25) (end 124.75 108.75) (width 0.3) (layer "F.Cu") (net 12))
 (segment (start 130.241 97.009) (end 130.241 96.30295) (width 0.3) (layer "F.Cu") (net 12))
 (segment (start 145 102) (end 145 105) (width 0.3) (layer "F.Cu") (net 20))
 (segment (start 162 78) (end 162 96.75) (width 0.3) (layer "F.Cu") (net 20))
 (segment (start 159.25 99.5) (end 147.5 99.5) (width 0.3) (layer "F.Cu") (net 20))
 (segment (start 141.75 108.25) (end 136.025 108.25) (width 0.3) (layer "F.Cu") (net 20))
 (segment (start 145 105) (end 141.75 108.25) (width 0.3) (layer "F.Cu") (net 20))
 (segment (start 147.5 99.5) (end 145 102) (width 0.3) (layer "F.Cu") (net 20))
 (segment (start 162 96.75) (end 159.25 99.5) (width 0.3) (layer "F.Cu") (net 20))
 (segment (start 146.92 73.57) (end 149.85 76.5) (width 0.3) (layer "F.Cu") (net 20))
 (segment (start 160.5 76.5) (end 162 78) (width 0.3) (layer "F.Cu") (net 20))
 (segment (start 149.85 76.5) (end 160.5 76.5) (width 0.3) (layer "F.Cu") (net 20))
 (segment (start 141.84 73.57) (end 141.84 74.63066) (width 0.3) (layer "F.Cu") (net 10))
 (segment (start 140.22066 76.25) (end 116.25 76.25) (width 0.3) (layer "F.Cu") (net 10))
 (segment (start 141.84 74.63066) (end 140.22066 76.25) (width 0.3) (layer "F.Cu") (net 10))
 (segment (start 115.75 106.5) (end 119.5 110.25) (width 0.3) (layer "F.Cu") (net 10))
 (segment (start 116.25 76.25) (end 115.75 76.75) (width 0.3) (layer "F.Cu") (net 10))
 (segment (start 119.5 110.25) (end 120.975 110.25) (width 0.3) (layer "F.Cu") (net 10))
 (segment (start 115.75 76.75) (end 115.75 106.5) (width 0.3) (layer "F.Cu") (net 10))
 (segment (start 125.75 109) (end 125.75 112.95) (width 0.3) (layer "F.Cu") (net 13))
 (segment (start 131.15 99.5) (end 131.15 103.6) (width 0.3) (layer "F.Cu") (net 13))
 (segment (start 131.15 103.6) (end 125.75 109) (width 0.3) (layer "F.Cu") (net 13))
 (segment (start 134.22 96.43) (end 131.15 99.5) (width 0.3) (layer "F.Cu") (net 13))
 (segment (start 122.45 116.25) (end 120.975 116.25) (width 0.3) (layer "F.Cu") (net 13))
 (segment (start 125.75 112.95) (end 122.45 116.25) (width 0.3) (layer "F.Cu") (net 13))
 (segment (start 134.03 73.57) (end 134.22 73.57) (width 0.3) (layer "F.Cu") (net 6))
 (segment (start 124.75 64.29) (end 134.03 73.57) (width 0.3) (layer "F.Cu") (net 6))
 (segment (start 129.14 73.57) (end 128.039 72.469) (width 0.3) (layer "F.Cu") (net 2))
 (segment (start 119.554598 119.25) (end 125.79148 119.25) (width 0.3) (layer "F.Cu") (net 2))
 (segment (start 124.503 74.747) (end 115.335959 74.747) (width 0.3) (layer "F.Cu") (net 2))
 (segment (start 125.161 73.11395) (end 125.161 74.089) (width 0.3) (layer "F.Cu") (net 2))
 (segment (start 125.161 74.089) (end 124.503 74.747) (width 0.3) (layer "F.Cu") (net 2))
 (segment (start 113.75 113.445402) (end 119.554598 119.25) (width 0.3) (layer "F.Cu") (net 2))
 (segment (start 125.79148 119.25) (end 125.999 119.45752) (width 0.3) (layer "F.Cu") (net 2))
 (segment (start 123.148 130.560017) (end 123.939984 131.352) (width 0.3) (layer "F.Cu") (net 2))
 (segment (start 125.999 119.45752) (end 125.999 120.29248) (width 0.3) (layer "F.Cu") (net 2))
 (segment (start 128.148 131.352) (end 129.5 130) (width 0.3) (layer "F.Cu") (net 2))
 (segment (start 125.80595 72.469) (end 125.161 73.11395) (width 0.3) (layer "F.Cu") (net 2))
 (segment (start 123.148 123.14348) (end 123.148 130.560017) (width 0.3) (layer "F.Cu") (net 2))
 (segment (start 123.939984 131.352) (end 128.148 131.352) (width 0.3) (layer "F.Cu") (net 2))
 (segment (start 113.75 76.332959) (end 113.75 113.445402) (width 0.3) (layer "F.Cu") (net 2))
 (segment (start 125.999 120.29248) (end 123.148 123.14348) (width 0.3) (layer "F.Cu") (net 2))
 (segment (start 115.335959 74.747) (end 113.75 76.332959) (width 0.3) (layer "F.Cu") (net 2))
 (segment (start 128.039 72.469) (end 125.80595 72.469) (width 0.3) (layer "F.Cu") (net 2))
 (segment (start 124.922 75.248) (end 126.6 73.57) (width 0.3) (layer "F.Cu") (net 3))
 (segment (start 124.5 117.25) (end 119.554598 117.25) (width 0.3) (layer "F.Cu") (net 3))
 (segment (start 118.5 112.25) (end 114.499 108.249) (width 0.3) (layer "F.Cu") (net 3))
 (segment (start 114.499 108.249) (end 114.499 76.292479) (width 0.3) (layer "F.Cu") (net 3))
 (segment (start 114.499 76.292479) (end 115.54348 75.248) (width 0.3) (layer "F.Cu") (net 3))
 (segment (start 126.5 119.25) (end 124.5 117.25) (width 0.3) (layer "F.Cu") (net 3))
 (segment (start 123.649 123.351) (end 126.5 120.5) (width 0.3) (layer "F.Cu") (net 3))
 (segment (start 124.147504 130.851) (end 123.649 130.352496) (width 0.3) (layer "F.Cu") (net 3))
 (segment (start 126.5 120.5) (end 126.5 119.25) (width 0.3) (layer "F.Cu") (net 3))
 (segment (start 115.54348 75.248) (end 124.922 75.248) (width 0.3) (layer "F.Cu") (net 3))
 (segment (start 119.554598 117.25) (end 118.5 116.195402) (width 0.3) (layer "F.Cu") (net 3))
 (segment (start 127 130) (end 126.149 130.851) (width 0.3) (layer "F.Cu") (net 3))
 (segment (start 118.5 116.195402) (end 118.5 112.25) (width 0.3) (layer "F.Cu") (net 3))
 (segment (start 126.149 130.851) (end 124.147504 130.851) (width 0.3) (layer "F.Cu") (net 3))
 (segment (start 123.649 130.352496) (end 123.649 123.351) (width 0.3) (layer "F.Cu") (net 3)))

